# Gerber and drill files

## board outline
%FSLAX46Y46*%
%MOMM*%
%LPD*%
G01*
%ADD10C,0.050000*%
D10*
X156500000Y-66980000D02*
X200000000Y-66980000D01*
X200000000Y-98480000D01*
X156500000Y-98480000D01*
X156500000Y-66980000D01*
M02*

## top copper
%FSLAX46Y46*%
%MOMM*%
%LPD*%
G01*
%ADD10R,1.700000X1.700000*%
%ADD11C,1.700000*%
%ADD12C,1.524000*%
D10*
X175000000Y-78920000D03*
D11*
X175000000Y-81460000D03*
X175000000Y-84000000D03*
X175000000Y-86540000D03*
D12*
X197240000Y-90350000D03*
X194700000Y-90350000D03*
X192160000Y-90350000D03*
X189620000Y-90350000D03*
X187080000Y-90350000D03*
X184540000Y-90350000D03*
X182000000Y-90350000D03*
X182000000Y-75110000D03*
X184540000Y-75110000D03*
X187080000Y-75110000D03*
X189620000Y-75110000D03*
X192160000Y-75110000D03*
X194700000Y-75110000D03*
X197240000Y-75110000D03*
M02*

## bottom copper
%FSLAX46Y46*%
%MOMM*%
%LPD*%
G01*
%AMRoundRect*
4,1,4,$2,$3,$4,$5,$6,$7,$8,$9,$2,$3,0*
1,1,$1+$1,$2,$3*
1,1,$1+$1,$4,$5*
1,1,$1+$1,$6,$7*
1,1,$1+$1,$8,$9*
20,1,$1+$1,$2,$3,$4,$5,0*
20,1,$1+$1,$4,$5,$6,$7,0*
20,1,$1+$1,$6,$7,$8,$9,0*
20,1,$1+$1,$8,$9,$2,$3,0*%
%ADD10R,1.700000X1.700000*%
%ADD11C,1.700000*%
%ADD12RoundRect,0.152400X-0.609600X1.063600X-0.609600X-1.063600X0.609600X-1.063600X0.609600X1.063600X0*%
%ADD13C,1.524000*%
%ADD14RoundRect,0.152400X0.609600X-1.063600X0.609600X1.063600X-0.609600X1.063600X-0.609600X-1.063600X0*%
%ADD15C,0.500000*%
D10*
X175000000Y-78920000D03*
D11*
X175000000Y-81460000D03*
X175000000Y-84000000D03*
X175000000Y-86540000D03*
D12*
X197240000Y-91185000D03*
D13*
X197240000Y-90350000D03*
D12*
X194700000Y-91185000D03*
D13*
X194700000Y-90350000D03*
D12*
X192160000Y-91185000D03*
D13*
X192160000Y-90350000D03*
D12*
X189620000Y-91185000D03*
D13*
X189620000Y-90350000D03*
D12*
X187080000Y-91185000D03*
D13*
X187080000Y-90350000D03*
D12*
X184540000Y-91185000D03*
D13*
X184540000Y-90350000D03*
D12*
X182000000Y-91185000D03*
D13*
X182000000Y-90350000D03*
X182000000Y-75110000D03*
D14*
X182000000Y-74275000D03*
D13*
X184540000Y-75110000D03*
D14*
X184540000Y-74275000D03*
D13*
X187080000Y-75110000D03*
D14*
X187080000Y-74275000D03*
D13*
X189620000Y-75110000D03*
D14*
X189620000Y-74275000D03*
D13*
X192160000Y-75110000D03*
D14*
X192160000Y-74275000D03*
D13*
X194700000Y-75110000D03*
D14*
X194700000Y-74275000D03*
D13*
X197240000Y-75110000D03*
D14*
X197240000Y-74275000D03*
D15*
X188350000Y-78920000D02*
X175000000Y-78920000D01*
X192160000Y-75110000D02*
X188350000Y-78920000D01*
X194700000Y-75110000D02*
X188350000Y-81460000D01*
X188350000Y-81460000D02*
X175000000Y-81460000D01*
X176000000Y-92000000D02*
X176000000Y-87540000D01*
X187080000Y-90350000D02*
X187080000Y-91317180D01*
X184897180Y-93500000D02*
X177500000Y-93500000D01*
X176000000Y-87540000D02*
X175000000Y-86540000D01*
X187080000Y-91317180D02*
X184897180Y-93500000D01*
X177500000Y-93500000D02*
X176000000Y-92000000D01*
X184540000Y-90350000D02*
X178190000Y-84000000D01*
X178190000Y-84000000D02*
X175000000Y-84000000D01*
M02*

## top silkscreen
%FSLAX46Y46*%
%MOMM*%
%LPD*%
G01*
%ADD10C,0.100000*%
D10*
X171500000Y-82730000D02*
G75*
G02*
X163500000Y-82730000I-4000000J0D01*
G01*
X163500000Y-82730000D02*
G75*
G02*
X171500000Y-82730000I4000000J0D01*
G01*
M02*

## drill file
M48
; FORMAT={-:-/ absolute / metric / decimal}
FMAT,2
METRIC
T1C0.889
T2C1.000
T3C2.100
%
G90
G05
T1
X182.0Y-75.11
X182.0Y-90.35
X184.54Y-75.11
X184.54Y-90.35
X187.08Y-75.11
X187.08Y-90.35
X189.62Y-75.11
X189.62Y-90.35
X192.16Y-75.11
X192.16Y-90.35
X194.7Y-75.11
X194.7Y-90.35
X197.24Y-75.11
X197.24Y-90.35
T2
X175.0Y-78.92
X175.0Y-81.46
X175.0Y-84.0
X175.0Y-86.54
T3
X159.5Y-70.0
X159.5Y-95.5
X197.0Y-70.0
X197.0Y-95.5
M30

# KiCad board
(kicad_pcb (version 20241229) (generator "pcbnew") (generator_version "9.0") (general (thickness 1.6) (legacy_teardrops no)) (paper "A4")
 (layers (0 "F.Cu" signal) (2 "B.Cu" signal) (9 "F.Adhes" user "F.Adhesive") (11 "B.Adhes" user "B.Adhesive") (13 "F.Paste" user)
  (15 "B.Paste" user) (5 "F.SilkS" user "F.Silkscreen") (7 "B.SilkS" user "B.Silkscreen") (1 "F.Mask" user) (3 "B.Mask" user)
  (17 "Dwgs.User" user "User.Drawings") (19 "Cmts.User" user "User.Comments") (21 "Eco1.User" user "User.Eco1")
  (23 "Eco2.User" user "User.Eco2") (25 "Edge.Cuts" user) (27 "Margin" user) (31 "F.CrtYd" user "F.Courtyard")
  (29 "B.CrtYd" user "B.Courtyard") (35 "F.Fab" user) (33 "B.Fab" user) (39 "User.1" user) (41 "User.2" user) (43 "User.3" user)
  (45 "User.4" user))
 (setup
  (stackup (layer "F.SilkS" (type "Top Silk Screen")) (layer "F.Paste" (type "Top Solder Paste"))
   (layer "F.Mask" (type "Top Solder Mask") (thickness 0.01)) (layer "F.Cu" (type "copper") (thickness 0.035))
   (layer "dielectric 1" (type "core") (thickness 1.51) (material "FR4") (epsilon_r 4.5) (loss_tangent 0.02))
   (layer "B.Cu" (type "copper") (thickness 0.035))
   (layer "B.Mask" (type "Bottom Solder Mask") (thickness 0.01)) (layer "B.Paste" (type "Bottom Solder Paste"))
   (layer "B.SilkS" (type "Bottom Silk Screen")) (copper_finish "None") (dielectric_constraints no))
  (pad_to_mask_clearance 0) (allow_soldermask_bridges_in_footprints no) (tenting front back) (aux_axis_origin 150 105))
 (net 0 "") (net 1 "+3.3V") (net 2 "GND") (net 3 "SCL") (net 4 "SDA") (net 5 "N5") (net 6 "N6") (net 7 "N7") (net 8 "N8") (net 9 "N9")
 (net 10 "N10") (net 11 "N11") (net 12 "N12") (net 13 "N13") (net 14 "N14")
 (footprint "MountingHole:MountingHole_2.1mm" (layer "F.Cu") (at 197 95.5)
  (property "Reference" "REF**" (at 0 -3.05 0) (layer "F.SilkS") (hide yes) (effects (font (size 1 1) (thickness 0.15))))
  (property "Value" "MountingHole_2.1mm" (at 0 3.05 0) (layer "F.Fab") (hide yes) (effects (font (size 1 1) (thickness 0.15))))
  (pad "" np_thru_hole circle (at 0 0) (size 2.1 2.1) (drill 2.1) (layers "*.Cu" "*.Mask")))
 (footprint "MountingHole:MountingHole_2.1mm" (layer "F.Cu") (at 197 70)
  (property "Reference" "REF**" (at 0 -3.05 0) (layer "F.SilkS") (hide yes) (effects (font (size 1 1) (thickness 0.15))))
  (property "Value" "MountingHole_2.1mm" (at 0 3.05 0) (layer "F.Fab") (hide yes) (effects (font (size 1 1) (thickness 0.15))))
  (pad "" np_thru_hole circle (at 0 0) (size 2.1 2.1) (drill 2.1) (layers "*.Cu" "*.Mask")))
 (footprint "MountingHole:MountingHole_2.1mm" (layer "F.Cu") (at 159.5 70)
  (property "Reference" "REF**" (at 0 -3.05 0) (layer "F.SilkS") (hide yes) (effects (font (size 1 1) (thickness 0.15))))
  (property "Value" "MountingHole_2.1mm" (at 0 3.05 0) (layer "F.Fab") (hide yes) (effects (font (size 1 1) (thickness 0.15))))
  (pad "" np_thru_hole circle (at 0 0) (size 2.1 2.1) (drill 2.1) (layers "*.Cu" "*.Mask")))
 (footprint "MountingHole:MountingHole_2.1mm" (layer "F.Cu") (at 159.5 95.5)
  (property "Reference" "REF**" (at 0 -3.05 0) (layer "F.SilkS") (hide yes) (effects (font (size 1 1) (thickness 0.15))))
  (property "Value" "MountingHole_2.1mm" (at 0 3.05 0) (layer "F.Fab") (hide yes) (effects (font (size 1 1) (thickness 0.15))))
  (pad "" np_thru_hole circle (at 0 0) (size 2.1 2.1) (drill 2.1) (layers "*.Cu" "*.Mask")))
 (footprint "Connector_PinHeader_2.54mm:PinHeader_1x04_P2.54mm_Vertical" (layer "B.Cu") (at 175 78.92 180)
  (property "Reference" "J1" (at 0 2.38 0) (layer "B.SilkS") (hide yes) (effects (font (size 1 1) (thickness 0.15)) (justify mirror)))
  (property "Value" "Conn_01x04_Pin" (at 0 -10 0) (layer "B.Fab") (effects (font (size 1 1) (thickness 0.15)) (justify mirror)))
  (pad "1" thru_hole rect (at 0 0 180) (size 1.7 1.7) (drill 1) (layers "*.Cu" "*.Mask") (remove_unused_layers no) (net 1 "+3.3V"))
  (pad "2" thru_hole circle (at 0 -2.54 180) (size 1.7 1.7) (drill 1) (layers "*.Cu" "*.Mask") (remove_unused_layers no) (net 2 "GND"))
  (pad "3" thru_hole circle (at 0 -5.08 180) (size 1.7 1.7) (drill 1) (layers "*.Cu" "*.Mask") (remove_unused_layers no) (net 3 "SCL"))
  (pad "4" thru_hole circle (at 0 -7.62 180) (size 1.7 1.7) (drill 1) (layers "*.Cu" "*.Mask") (remove_unused_layers no) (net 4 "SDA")))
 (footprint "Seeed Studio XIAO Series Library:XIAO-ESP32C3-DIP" (layer "B.Cu") (at 189.62 82.61 90)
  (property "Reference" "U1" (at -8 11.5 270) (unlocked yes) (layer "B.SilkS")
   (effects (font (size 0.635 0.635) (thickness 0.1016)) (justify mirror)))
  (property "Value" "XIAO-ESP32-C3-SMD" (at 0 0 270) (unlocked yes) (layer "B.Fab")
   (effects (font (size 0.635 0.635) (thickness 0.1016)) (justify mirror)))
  (pad "1" smd roundrect (at -8.575 7.62 270) (size 2.432 1.524) (layers "B.Cu" "B.Mask") (roundrect_rratio 0.1) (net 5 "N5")
   (thermal_bridge_angle 45))
  (pad "1" thru_hole circle (at -7.74 7.62 270) (size 1.524 1.524) (drill 0.889) (layers "*.Cu" "*.Mask") (remove_unused_layers no)
   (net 5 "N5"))
  (pad "2" smd roundrect (at -8.575 5.08 270) (size 2.432 1.524) (layers "B.Cu" "B.Mask") (roundrect_rratio 0.1) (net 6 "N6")
   (thermal_bridge_angle 45))
  (pad "2" thru_hole circle (at -7.74 5.08 270) (size 1.524 1.524) (drill 0.889) (layers "*.Cu" "*.Mask") (remove_unused_layers no)
   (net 6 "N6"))
  (pad "3" smd roundrect (at -8.575 2.54 270) (size 2.432 1.524) (layers "B.Cu" "B.Mask") (roundrect_rratio 0.1) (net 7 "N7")
   (thermal_bridge_angle 45))
  (pad "3" thru_hole circle (at -7.74 2.54 270) (size 1.524 1.524) (drill 0.889) (layers "*.Cu" "*.Mask") (remove_unused_layers no)
   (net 7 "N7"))
  (pad "4" smd roundrect (at -8.575 0 270) (size 2.432 1.524) (layers "B.Cu" "B.Mask") (roundrect_rratio 0.1) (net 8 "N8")
   (thermal_bridge_angle 45))
  (pad "4" thru_hole circle (at -7.74 0 270) (size 1.524 1.524) (drill 0.889) (layers "*.Cu" "*.Mask") (remove_unused_layers no)
   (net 8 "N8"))
  (pad "5" smd roundrect (at -8.575 -2.54 270) (size 2.432 1.524) (layers "B.Cu" "B.Mask") (roundrect_rratio 0.1) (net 4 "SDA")
   (thermal_bridge_angle 45))
  (pad "5" thru_hole circle (at -7.74 -2.54 270) (size 1.524 1.524) (drill 0.889) (layers "*.Cu" "*.Mask") (remove_unused_layers no)
   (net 4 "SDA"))
  (pad "6" smd roundrect (at -8.575 -5.08 270) (size 2.432 1.524) (layers "B.Cu" "B.Mask") (roundrect_rratio 0.1) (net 3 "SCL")
   (thermal_bridge_angle 45))
  (pad "6" thru_hole circle (at -7.74 -5.08 270) (size 1.524 1.524) (drill 0.889) (layers "*.Cu" "*.Mask") (remove_unused_layers no)
   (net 3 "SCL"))
  (pad "7" smd roundrect (at -8.575 -7.62 270) (size 2.432 1.524) (layers "B.Cu" "B.Mask") (roundrect_rratio 0.1) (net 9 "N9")
   (thermal_bridge_angle 45))
  (pad "7" thru_hole circle (at -7.74 -7.62 270) (size 1.524 1.524) (drill 0.889) (layers "*.Cu" "*.Mask") (remove_unused_layers no)
   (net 9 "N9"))
  (pad "8" thru_hole circle (at 7.5 -7.62 90) (size 1.524 1.524) (drill 0.889) (layers "*.Cu" "*.Mask") (remove_unused_layers no)
   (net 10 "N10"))
  (pad "8" smd roundrect (at 8.335 -7.62 90) (size 2.432 1.524) (layers "B.Cu" "B.Mask") (roundrect_rratio 0.1) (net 10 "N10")
   (thermal_bridge_angle 45))
  (pad "9" thru_hole circle (at 7.5 -5.08 90) (size 1.524 1.524) (drill 0.889) (layers "*.Cu" "*.Mask") (remove_unused_layers no)
   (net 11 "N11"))
  (pad "9" smd roundrect (at 8.335 -5.08 90) (size 2.432 1.524) (layers "B.Cu" "B.Mask") (roundrect_rratio 0.1) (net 11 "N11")
   (thermal_bridge_angle 45))
  (pad "10" thru_hole circle (at 7.5 -2.54 90) (size 1.524 1.524) (drill 0.889) (layers "*.Cu" "*.Mask") (remove_unused_layers no)
   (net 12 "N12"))
  (pad "10" smd roundrect (at 8.335 -2.54 90) (size 2.432 1.524) (layers "B.Cu" "B.Mask") (roundrect_rratio 0.1) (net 12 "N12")
   (thermal_bridge_angle 45))
  (pad "11" thru_hole circle (at 7.5 0 90) (size 1.524 1.524) (drill 0.889) (layers "*.Cu" "*.Mask") (remove_unused_layers no)
   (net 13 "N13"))
  (pad "11" smd roundrect (at 8.335 0 90) (size 2.432 1.524) (layers "B.Cu" "B.Mask") (roundrect_rratio 0.1) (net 13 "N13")
   (thermal_bridge_angle 45))
  (pad "12" thru_hole circle (at 7.5 2.54 90) (size 1.524 1.524) (drill 0.889) (layers "*.Cu" "*.Mask") (remove_unused_layers no)
   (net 1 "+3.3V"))
  (pad "12" smd roundrect (at 8.335 2.54 90) (size 2.432 1.524) (layers "B.Cu" "B.Mask") (roundrect_rratio 0.1) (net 1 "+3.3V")
   (thermal_bridge_angle 45))
  (pad "13" thru_hole circle (at 7.5 5.08 90) (size 1.524 1.524) (drill 0.889) (layers "*.Cu" "*.Mask") (remove_unused_layers no)
   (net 2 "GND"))
  (pad "13" smd roundrect (at 8.335 5.08 90) (size 2.432 1.524) (layers "B.Cu" "B.Mask") (roundrect_rratio 0.1) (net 2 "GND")
   (thermal_bridge_angle 45))
  (pad "14" thru_hole circle (at 7.5 7.62 90) (size 1.524 1.524) (drill 0.889) (layers "*.Cu" "*.Mask") (remove_unused_layers no)
   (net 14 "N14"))
  (pad "14" smd roundrect (at 8.335 7.62 90) (size 2.432 1.524) (layers "B.Cu" "B.Mask") (roundrect_rratio 0.1) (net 14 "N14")
   (thermal_bridge_angle 45)))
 (gr_circle (center 167.5 82.73) (end 163.5 82.73) (stroke (width 0.1) (type solid)) (fill no) (layer "F.SilkS"))
 (gr_rect (start 156.5 66.98) (end 200 98.48) (stroke (width 0.05) (type default)) (fill no) (layer "Edge.Cuts"))
 (segment (start 188.35 78.92) (end 175 78.92) (width 0.5) (layer "B.Cu") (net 1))
 (segment (start 192.16 75.11) (end 188.35 78.92) (width 0.5) (layer "B.Cu") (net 1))
 (segment (start 194.7 75.11) (end 188.35 81.46) (width 0.5) (layer "B.Cu") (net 2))
 (segment (start 188.35 81.46) (end 175 81.46) (width 0.5) (layer "B.Cu") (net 2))
 (segment (start 176 92) (end 176 87.54) (width 0.5) (layer "B.Cu") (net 4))
 (segment (start 187.08 90.35) (end 187.08 91.31718) (width 0.5) (layer "B.Cu") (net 4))
 (segment (start 184.89718 93.5) (end 177.5 93.5) (width 0.5) (layer "B.Cu") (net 4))
 (segment (start 176 87.54) (end 175 86.54) (width 0.5) (layer "B.Cu") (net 4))
 (segment (start 187.08 91.31718) (end 184.89718 93.5) (width 0.5) (layer "B.Cu") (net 4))
 (segment (start 177.5 93.5) (end 176 92) (width 0.5) (layer "B.Cu") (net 4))
 (segment (start 184.54 90.35) (end 178.19 84) (width 0.5) (layer "B.Cu") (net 3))
 (segment (start 178.19 84) (end 175 84) (width 0.5) (layer "B.Cu") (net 3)))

